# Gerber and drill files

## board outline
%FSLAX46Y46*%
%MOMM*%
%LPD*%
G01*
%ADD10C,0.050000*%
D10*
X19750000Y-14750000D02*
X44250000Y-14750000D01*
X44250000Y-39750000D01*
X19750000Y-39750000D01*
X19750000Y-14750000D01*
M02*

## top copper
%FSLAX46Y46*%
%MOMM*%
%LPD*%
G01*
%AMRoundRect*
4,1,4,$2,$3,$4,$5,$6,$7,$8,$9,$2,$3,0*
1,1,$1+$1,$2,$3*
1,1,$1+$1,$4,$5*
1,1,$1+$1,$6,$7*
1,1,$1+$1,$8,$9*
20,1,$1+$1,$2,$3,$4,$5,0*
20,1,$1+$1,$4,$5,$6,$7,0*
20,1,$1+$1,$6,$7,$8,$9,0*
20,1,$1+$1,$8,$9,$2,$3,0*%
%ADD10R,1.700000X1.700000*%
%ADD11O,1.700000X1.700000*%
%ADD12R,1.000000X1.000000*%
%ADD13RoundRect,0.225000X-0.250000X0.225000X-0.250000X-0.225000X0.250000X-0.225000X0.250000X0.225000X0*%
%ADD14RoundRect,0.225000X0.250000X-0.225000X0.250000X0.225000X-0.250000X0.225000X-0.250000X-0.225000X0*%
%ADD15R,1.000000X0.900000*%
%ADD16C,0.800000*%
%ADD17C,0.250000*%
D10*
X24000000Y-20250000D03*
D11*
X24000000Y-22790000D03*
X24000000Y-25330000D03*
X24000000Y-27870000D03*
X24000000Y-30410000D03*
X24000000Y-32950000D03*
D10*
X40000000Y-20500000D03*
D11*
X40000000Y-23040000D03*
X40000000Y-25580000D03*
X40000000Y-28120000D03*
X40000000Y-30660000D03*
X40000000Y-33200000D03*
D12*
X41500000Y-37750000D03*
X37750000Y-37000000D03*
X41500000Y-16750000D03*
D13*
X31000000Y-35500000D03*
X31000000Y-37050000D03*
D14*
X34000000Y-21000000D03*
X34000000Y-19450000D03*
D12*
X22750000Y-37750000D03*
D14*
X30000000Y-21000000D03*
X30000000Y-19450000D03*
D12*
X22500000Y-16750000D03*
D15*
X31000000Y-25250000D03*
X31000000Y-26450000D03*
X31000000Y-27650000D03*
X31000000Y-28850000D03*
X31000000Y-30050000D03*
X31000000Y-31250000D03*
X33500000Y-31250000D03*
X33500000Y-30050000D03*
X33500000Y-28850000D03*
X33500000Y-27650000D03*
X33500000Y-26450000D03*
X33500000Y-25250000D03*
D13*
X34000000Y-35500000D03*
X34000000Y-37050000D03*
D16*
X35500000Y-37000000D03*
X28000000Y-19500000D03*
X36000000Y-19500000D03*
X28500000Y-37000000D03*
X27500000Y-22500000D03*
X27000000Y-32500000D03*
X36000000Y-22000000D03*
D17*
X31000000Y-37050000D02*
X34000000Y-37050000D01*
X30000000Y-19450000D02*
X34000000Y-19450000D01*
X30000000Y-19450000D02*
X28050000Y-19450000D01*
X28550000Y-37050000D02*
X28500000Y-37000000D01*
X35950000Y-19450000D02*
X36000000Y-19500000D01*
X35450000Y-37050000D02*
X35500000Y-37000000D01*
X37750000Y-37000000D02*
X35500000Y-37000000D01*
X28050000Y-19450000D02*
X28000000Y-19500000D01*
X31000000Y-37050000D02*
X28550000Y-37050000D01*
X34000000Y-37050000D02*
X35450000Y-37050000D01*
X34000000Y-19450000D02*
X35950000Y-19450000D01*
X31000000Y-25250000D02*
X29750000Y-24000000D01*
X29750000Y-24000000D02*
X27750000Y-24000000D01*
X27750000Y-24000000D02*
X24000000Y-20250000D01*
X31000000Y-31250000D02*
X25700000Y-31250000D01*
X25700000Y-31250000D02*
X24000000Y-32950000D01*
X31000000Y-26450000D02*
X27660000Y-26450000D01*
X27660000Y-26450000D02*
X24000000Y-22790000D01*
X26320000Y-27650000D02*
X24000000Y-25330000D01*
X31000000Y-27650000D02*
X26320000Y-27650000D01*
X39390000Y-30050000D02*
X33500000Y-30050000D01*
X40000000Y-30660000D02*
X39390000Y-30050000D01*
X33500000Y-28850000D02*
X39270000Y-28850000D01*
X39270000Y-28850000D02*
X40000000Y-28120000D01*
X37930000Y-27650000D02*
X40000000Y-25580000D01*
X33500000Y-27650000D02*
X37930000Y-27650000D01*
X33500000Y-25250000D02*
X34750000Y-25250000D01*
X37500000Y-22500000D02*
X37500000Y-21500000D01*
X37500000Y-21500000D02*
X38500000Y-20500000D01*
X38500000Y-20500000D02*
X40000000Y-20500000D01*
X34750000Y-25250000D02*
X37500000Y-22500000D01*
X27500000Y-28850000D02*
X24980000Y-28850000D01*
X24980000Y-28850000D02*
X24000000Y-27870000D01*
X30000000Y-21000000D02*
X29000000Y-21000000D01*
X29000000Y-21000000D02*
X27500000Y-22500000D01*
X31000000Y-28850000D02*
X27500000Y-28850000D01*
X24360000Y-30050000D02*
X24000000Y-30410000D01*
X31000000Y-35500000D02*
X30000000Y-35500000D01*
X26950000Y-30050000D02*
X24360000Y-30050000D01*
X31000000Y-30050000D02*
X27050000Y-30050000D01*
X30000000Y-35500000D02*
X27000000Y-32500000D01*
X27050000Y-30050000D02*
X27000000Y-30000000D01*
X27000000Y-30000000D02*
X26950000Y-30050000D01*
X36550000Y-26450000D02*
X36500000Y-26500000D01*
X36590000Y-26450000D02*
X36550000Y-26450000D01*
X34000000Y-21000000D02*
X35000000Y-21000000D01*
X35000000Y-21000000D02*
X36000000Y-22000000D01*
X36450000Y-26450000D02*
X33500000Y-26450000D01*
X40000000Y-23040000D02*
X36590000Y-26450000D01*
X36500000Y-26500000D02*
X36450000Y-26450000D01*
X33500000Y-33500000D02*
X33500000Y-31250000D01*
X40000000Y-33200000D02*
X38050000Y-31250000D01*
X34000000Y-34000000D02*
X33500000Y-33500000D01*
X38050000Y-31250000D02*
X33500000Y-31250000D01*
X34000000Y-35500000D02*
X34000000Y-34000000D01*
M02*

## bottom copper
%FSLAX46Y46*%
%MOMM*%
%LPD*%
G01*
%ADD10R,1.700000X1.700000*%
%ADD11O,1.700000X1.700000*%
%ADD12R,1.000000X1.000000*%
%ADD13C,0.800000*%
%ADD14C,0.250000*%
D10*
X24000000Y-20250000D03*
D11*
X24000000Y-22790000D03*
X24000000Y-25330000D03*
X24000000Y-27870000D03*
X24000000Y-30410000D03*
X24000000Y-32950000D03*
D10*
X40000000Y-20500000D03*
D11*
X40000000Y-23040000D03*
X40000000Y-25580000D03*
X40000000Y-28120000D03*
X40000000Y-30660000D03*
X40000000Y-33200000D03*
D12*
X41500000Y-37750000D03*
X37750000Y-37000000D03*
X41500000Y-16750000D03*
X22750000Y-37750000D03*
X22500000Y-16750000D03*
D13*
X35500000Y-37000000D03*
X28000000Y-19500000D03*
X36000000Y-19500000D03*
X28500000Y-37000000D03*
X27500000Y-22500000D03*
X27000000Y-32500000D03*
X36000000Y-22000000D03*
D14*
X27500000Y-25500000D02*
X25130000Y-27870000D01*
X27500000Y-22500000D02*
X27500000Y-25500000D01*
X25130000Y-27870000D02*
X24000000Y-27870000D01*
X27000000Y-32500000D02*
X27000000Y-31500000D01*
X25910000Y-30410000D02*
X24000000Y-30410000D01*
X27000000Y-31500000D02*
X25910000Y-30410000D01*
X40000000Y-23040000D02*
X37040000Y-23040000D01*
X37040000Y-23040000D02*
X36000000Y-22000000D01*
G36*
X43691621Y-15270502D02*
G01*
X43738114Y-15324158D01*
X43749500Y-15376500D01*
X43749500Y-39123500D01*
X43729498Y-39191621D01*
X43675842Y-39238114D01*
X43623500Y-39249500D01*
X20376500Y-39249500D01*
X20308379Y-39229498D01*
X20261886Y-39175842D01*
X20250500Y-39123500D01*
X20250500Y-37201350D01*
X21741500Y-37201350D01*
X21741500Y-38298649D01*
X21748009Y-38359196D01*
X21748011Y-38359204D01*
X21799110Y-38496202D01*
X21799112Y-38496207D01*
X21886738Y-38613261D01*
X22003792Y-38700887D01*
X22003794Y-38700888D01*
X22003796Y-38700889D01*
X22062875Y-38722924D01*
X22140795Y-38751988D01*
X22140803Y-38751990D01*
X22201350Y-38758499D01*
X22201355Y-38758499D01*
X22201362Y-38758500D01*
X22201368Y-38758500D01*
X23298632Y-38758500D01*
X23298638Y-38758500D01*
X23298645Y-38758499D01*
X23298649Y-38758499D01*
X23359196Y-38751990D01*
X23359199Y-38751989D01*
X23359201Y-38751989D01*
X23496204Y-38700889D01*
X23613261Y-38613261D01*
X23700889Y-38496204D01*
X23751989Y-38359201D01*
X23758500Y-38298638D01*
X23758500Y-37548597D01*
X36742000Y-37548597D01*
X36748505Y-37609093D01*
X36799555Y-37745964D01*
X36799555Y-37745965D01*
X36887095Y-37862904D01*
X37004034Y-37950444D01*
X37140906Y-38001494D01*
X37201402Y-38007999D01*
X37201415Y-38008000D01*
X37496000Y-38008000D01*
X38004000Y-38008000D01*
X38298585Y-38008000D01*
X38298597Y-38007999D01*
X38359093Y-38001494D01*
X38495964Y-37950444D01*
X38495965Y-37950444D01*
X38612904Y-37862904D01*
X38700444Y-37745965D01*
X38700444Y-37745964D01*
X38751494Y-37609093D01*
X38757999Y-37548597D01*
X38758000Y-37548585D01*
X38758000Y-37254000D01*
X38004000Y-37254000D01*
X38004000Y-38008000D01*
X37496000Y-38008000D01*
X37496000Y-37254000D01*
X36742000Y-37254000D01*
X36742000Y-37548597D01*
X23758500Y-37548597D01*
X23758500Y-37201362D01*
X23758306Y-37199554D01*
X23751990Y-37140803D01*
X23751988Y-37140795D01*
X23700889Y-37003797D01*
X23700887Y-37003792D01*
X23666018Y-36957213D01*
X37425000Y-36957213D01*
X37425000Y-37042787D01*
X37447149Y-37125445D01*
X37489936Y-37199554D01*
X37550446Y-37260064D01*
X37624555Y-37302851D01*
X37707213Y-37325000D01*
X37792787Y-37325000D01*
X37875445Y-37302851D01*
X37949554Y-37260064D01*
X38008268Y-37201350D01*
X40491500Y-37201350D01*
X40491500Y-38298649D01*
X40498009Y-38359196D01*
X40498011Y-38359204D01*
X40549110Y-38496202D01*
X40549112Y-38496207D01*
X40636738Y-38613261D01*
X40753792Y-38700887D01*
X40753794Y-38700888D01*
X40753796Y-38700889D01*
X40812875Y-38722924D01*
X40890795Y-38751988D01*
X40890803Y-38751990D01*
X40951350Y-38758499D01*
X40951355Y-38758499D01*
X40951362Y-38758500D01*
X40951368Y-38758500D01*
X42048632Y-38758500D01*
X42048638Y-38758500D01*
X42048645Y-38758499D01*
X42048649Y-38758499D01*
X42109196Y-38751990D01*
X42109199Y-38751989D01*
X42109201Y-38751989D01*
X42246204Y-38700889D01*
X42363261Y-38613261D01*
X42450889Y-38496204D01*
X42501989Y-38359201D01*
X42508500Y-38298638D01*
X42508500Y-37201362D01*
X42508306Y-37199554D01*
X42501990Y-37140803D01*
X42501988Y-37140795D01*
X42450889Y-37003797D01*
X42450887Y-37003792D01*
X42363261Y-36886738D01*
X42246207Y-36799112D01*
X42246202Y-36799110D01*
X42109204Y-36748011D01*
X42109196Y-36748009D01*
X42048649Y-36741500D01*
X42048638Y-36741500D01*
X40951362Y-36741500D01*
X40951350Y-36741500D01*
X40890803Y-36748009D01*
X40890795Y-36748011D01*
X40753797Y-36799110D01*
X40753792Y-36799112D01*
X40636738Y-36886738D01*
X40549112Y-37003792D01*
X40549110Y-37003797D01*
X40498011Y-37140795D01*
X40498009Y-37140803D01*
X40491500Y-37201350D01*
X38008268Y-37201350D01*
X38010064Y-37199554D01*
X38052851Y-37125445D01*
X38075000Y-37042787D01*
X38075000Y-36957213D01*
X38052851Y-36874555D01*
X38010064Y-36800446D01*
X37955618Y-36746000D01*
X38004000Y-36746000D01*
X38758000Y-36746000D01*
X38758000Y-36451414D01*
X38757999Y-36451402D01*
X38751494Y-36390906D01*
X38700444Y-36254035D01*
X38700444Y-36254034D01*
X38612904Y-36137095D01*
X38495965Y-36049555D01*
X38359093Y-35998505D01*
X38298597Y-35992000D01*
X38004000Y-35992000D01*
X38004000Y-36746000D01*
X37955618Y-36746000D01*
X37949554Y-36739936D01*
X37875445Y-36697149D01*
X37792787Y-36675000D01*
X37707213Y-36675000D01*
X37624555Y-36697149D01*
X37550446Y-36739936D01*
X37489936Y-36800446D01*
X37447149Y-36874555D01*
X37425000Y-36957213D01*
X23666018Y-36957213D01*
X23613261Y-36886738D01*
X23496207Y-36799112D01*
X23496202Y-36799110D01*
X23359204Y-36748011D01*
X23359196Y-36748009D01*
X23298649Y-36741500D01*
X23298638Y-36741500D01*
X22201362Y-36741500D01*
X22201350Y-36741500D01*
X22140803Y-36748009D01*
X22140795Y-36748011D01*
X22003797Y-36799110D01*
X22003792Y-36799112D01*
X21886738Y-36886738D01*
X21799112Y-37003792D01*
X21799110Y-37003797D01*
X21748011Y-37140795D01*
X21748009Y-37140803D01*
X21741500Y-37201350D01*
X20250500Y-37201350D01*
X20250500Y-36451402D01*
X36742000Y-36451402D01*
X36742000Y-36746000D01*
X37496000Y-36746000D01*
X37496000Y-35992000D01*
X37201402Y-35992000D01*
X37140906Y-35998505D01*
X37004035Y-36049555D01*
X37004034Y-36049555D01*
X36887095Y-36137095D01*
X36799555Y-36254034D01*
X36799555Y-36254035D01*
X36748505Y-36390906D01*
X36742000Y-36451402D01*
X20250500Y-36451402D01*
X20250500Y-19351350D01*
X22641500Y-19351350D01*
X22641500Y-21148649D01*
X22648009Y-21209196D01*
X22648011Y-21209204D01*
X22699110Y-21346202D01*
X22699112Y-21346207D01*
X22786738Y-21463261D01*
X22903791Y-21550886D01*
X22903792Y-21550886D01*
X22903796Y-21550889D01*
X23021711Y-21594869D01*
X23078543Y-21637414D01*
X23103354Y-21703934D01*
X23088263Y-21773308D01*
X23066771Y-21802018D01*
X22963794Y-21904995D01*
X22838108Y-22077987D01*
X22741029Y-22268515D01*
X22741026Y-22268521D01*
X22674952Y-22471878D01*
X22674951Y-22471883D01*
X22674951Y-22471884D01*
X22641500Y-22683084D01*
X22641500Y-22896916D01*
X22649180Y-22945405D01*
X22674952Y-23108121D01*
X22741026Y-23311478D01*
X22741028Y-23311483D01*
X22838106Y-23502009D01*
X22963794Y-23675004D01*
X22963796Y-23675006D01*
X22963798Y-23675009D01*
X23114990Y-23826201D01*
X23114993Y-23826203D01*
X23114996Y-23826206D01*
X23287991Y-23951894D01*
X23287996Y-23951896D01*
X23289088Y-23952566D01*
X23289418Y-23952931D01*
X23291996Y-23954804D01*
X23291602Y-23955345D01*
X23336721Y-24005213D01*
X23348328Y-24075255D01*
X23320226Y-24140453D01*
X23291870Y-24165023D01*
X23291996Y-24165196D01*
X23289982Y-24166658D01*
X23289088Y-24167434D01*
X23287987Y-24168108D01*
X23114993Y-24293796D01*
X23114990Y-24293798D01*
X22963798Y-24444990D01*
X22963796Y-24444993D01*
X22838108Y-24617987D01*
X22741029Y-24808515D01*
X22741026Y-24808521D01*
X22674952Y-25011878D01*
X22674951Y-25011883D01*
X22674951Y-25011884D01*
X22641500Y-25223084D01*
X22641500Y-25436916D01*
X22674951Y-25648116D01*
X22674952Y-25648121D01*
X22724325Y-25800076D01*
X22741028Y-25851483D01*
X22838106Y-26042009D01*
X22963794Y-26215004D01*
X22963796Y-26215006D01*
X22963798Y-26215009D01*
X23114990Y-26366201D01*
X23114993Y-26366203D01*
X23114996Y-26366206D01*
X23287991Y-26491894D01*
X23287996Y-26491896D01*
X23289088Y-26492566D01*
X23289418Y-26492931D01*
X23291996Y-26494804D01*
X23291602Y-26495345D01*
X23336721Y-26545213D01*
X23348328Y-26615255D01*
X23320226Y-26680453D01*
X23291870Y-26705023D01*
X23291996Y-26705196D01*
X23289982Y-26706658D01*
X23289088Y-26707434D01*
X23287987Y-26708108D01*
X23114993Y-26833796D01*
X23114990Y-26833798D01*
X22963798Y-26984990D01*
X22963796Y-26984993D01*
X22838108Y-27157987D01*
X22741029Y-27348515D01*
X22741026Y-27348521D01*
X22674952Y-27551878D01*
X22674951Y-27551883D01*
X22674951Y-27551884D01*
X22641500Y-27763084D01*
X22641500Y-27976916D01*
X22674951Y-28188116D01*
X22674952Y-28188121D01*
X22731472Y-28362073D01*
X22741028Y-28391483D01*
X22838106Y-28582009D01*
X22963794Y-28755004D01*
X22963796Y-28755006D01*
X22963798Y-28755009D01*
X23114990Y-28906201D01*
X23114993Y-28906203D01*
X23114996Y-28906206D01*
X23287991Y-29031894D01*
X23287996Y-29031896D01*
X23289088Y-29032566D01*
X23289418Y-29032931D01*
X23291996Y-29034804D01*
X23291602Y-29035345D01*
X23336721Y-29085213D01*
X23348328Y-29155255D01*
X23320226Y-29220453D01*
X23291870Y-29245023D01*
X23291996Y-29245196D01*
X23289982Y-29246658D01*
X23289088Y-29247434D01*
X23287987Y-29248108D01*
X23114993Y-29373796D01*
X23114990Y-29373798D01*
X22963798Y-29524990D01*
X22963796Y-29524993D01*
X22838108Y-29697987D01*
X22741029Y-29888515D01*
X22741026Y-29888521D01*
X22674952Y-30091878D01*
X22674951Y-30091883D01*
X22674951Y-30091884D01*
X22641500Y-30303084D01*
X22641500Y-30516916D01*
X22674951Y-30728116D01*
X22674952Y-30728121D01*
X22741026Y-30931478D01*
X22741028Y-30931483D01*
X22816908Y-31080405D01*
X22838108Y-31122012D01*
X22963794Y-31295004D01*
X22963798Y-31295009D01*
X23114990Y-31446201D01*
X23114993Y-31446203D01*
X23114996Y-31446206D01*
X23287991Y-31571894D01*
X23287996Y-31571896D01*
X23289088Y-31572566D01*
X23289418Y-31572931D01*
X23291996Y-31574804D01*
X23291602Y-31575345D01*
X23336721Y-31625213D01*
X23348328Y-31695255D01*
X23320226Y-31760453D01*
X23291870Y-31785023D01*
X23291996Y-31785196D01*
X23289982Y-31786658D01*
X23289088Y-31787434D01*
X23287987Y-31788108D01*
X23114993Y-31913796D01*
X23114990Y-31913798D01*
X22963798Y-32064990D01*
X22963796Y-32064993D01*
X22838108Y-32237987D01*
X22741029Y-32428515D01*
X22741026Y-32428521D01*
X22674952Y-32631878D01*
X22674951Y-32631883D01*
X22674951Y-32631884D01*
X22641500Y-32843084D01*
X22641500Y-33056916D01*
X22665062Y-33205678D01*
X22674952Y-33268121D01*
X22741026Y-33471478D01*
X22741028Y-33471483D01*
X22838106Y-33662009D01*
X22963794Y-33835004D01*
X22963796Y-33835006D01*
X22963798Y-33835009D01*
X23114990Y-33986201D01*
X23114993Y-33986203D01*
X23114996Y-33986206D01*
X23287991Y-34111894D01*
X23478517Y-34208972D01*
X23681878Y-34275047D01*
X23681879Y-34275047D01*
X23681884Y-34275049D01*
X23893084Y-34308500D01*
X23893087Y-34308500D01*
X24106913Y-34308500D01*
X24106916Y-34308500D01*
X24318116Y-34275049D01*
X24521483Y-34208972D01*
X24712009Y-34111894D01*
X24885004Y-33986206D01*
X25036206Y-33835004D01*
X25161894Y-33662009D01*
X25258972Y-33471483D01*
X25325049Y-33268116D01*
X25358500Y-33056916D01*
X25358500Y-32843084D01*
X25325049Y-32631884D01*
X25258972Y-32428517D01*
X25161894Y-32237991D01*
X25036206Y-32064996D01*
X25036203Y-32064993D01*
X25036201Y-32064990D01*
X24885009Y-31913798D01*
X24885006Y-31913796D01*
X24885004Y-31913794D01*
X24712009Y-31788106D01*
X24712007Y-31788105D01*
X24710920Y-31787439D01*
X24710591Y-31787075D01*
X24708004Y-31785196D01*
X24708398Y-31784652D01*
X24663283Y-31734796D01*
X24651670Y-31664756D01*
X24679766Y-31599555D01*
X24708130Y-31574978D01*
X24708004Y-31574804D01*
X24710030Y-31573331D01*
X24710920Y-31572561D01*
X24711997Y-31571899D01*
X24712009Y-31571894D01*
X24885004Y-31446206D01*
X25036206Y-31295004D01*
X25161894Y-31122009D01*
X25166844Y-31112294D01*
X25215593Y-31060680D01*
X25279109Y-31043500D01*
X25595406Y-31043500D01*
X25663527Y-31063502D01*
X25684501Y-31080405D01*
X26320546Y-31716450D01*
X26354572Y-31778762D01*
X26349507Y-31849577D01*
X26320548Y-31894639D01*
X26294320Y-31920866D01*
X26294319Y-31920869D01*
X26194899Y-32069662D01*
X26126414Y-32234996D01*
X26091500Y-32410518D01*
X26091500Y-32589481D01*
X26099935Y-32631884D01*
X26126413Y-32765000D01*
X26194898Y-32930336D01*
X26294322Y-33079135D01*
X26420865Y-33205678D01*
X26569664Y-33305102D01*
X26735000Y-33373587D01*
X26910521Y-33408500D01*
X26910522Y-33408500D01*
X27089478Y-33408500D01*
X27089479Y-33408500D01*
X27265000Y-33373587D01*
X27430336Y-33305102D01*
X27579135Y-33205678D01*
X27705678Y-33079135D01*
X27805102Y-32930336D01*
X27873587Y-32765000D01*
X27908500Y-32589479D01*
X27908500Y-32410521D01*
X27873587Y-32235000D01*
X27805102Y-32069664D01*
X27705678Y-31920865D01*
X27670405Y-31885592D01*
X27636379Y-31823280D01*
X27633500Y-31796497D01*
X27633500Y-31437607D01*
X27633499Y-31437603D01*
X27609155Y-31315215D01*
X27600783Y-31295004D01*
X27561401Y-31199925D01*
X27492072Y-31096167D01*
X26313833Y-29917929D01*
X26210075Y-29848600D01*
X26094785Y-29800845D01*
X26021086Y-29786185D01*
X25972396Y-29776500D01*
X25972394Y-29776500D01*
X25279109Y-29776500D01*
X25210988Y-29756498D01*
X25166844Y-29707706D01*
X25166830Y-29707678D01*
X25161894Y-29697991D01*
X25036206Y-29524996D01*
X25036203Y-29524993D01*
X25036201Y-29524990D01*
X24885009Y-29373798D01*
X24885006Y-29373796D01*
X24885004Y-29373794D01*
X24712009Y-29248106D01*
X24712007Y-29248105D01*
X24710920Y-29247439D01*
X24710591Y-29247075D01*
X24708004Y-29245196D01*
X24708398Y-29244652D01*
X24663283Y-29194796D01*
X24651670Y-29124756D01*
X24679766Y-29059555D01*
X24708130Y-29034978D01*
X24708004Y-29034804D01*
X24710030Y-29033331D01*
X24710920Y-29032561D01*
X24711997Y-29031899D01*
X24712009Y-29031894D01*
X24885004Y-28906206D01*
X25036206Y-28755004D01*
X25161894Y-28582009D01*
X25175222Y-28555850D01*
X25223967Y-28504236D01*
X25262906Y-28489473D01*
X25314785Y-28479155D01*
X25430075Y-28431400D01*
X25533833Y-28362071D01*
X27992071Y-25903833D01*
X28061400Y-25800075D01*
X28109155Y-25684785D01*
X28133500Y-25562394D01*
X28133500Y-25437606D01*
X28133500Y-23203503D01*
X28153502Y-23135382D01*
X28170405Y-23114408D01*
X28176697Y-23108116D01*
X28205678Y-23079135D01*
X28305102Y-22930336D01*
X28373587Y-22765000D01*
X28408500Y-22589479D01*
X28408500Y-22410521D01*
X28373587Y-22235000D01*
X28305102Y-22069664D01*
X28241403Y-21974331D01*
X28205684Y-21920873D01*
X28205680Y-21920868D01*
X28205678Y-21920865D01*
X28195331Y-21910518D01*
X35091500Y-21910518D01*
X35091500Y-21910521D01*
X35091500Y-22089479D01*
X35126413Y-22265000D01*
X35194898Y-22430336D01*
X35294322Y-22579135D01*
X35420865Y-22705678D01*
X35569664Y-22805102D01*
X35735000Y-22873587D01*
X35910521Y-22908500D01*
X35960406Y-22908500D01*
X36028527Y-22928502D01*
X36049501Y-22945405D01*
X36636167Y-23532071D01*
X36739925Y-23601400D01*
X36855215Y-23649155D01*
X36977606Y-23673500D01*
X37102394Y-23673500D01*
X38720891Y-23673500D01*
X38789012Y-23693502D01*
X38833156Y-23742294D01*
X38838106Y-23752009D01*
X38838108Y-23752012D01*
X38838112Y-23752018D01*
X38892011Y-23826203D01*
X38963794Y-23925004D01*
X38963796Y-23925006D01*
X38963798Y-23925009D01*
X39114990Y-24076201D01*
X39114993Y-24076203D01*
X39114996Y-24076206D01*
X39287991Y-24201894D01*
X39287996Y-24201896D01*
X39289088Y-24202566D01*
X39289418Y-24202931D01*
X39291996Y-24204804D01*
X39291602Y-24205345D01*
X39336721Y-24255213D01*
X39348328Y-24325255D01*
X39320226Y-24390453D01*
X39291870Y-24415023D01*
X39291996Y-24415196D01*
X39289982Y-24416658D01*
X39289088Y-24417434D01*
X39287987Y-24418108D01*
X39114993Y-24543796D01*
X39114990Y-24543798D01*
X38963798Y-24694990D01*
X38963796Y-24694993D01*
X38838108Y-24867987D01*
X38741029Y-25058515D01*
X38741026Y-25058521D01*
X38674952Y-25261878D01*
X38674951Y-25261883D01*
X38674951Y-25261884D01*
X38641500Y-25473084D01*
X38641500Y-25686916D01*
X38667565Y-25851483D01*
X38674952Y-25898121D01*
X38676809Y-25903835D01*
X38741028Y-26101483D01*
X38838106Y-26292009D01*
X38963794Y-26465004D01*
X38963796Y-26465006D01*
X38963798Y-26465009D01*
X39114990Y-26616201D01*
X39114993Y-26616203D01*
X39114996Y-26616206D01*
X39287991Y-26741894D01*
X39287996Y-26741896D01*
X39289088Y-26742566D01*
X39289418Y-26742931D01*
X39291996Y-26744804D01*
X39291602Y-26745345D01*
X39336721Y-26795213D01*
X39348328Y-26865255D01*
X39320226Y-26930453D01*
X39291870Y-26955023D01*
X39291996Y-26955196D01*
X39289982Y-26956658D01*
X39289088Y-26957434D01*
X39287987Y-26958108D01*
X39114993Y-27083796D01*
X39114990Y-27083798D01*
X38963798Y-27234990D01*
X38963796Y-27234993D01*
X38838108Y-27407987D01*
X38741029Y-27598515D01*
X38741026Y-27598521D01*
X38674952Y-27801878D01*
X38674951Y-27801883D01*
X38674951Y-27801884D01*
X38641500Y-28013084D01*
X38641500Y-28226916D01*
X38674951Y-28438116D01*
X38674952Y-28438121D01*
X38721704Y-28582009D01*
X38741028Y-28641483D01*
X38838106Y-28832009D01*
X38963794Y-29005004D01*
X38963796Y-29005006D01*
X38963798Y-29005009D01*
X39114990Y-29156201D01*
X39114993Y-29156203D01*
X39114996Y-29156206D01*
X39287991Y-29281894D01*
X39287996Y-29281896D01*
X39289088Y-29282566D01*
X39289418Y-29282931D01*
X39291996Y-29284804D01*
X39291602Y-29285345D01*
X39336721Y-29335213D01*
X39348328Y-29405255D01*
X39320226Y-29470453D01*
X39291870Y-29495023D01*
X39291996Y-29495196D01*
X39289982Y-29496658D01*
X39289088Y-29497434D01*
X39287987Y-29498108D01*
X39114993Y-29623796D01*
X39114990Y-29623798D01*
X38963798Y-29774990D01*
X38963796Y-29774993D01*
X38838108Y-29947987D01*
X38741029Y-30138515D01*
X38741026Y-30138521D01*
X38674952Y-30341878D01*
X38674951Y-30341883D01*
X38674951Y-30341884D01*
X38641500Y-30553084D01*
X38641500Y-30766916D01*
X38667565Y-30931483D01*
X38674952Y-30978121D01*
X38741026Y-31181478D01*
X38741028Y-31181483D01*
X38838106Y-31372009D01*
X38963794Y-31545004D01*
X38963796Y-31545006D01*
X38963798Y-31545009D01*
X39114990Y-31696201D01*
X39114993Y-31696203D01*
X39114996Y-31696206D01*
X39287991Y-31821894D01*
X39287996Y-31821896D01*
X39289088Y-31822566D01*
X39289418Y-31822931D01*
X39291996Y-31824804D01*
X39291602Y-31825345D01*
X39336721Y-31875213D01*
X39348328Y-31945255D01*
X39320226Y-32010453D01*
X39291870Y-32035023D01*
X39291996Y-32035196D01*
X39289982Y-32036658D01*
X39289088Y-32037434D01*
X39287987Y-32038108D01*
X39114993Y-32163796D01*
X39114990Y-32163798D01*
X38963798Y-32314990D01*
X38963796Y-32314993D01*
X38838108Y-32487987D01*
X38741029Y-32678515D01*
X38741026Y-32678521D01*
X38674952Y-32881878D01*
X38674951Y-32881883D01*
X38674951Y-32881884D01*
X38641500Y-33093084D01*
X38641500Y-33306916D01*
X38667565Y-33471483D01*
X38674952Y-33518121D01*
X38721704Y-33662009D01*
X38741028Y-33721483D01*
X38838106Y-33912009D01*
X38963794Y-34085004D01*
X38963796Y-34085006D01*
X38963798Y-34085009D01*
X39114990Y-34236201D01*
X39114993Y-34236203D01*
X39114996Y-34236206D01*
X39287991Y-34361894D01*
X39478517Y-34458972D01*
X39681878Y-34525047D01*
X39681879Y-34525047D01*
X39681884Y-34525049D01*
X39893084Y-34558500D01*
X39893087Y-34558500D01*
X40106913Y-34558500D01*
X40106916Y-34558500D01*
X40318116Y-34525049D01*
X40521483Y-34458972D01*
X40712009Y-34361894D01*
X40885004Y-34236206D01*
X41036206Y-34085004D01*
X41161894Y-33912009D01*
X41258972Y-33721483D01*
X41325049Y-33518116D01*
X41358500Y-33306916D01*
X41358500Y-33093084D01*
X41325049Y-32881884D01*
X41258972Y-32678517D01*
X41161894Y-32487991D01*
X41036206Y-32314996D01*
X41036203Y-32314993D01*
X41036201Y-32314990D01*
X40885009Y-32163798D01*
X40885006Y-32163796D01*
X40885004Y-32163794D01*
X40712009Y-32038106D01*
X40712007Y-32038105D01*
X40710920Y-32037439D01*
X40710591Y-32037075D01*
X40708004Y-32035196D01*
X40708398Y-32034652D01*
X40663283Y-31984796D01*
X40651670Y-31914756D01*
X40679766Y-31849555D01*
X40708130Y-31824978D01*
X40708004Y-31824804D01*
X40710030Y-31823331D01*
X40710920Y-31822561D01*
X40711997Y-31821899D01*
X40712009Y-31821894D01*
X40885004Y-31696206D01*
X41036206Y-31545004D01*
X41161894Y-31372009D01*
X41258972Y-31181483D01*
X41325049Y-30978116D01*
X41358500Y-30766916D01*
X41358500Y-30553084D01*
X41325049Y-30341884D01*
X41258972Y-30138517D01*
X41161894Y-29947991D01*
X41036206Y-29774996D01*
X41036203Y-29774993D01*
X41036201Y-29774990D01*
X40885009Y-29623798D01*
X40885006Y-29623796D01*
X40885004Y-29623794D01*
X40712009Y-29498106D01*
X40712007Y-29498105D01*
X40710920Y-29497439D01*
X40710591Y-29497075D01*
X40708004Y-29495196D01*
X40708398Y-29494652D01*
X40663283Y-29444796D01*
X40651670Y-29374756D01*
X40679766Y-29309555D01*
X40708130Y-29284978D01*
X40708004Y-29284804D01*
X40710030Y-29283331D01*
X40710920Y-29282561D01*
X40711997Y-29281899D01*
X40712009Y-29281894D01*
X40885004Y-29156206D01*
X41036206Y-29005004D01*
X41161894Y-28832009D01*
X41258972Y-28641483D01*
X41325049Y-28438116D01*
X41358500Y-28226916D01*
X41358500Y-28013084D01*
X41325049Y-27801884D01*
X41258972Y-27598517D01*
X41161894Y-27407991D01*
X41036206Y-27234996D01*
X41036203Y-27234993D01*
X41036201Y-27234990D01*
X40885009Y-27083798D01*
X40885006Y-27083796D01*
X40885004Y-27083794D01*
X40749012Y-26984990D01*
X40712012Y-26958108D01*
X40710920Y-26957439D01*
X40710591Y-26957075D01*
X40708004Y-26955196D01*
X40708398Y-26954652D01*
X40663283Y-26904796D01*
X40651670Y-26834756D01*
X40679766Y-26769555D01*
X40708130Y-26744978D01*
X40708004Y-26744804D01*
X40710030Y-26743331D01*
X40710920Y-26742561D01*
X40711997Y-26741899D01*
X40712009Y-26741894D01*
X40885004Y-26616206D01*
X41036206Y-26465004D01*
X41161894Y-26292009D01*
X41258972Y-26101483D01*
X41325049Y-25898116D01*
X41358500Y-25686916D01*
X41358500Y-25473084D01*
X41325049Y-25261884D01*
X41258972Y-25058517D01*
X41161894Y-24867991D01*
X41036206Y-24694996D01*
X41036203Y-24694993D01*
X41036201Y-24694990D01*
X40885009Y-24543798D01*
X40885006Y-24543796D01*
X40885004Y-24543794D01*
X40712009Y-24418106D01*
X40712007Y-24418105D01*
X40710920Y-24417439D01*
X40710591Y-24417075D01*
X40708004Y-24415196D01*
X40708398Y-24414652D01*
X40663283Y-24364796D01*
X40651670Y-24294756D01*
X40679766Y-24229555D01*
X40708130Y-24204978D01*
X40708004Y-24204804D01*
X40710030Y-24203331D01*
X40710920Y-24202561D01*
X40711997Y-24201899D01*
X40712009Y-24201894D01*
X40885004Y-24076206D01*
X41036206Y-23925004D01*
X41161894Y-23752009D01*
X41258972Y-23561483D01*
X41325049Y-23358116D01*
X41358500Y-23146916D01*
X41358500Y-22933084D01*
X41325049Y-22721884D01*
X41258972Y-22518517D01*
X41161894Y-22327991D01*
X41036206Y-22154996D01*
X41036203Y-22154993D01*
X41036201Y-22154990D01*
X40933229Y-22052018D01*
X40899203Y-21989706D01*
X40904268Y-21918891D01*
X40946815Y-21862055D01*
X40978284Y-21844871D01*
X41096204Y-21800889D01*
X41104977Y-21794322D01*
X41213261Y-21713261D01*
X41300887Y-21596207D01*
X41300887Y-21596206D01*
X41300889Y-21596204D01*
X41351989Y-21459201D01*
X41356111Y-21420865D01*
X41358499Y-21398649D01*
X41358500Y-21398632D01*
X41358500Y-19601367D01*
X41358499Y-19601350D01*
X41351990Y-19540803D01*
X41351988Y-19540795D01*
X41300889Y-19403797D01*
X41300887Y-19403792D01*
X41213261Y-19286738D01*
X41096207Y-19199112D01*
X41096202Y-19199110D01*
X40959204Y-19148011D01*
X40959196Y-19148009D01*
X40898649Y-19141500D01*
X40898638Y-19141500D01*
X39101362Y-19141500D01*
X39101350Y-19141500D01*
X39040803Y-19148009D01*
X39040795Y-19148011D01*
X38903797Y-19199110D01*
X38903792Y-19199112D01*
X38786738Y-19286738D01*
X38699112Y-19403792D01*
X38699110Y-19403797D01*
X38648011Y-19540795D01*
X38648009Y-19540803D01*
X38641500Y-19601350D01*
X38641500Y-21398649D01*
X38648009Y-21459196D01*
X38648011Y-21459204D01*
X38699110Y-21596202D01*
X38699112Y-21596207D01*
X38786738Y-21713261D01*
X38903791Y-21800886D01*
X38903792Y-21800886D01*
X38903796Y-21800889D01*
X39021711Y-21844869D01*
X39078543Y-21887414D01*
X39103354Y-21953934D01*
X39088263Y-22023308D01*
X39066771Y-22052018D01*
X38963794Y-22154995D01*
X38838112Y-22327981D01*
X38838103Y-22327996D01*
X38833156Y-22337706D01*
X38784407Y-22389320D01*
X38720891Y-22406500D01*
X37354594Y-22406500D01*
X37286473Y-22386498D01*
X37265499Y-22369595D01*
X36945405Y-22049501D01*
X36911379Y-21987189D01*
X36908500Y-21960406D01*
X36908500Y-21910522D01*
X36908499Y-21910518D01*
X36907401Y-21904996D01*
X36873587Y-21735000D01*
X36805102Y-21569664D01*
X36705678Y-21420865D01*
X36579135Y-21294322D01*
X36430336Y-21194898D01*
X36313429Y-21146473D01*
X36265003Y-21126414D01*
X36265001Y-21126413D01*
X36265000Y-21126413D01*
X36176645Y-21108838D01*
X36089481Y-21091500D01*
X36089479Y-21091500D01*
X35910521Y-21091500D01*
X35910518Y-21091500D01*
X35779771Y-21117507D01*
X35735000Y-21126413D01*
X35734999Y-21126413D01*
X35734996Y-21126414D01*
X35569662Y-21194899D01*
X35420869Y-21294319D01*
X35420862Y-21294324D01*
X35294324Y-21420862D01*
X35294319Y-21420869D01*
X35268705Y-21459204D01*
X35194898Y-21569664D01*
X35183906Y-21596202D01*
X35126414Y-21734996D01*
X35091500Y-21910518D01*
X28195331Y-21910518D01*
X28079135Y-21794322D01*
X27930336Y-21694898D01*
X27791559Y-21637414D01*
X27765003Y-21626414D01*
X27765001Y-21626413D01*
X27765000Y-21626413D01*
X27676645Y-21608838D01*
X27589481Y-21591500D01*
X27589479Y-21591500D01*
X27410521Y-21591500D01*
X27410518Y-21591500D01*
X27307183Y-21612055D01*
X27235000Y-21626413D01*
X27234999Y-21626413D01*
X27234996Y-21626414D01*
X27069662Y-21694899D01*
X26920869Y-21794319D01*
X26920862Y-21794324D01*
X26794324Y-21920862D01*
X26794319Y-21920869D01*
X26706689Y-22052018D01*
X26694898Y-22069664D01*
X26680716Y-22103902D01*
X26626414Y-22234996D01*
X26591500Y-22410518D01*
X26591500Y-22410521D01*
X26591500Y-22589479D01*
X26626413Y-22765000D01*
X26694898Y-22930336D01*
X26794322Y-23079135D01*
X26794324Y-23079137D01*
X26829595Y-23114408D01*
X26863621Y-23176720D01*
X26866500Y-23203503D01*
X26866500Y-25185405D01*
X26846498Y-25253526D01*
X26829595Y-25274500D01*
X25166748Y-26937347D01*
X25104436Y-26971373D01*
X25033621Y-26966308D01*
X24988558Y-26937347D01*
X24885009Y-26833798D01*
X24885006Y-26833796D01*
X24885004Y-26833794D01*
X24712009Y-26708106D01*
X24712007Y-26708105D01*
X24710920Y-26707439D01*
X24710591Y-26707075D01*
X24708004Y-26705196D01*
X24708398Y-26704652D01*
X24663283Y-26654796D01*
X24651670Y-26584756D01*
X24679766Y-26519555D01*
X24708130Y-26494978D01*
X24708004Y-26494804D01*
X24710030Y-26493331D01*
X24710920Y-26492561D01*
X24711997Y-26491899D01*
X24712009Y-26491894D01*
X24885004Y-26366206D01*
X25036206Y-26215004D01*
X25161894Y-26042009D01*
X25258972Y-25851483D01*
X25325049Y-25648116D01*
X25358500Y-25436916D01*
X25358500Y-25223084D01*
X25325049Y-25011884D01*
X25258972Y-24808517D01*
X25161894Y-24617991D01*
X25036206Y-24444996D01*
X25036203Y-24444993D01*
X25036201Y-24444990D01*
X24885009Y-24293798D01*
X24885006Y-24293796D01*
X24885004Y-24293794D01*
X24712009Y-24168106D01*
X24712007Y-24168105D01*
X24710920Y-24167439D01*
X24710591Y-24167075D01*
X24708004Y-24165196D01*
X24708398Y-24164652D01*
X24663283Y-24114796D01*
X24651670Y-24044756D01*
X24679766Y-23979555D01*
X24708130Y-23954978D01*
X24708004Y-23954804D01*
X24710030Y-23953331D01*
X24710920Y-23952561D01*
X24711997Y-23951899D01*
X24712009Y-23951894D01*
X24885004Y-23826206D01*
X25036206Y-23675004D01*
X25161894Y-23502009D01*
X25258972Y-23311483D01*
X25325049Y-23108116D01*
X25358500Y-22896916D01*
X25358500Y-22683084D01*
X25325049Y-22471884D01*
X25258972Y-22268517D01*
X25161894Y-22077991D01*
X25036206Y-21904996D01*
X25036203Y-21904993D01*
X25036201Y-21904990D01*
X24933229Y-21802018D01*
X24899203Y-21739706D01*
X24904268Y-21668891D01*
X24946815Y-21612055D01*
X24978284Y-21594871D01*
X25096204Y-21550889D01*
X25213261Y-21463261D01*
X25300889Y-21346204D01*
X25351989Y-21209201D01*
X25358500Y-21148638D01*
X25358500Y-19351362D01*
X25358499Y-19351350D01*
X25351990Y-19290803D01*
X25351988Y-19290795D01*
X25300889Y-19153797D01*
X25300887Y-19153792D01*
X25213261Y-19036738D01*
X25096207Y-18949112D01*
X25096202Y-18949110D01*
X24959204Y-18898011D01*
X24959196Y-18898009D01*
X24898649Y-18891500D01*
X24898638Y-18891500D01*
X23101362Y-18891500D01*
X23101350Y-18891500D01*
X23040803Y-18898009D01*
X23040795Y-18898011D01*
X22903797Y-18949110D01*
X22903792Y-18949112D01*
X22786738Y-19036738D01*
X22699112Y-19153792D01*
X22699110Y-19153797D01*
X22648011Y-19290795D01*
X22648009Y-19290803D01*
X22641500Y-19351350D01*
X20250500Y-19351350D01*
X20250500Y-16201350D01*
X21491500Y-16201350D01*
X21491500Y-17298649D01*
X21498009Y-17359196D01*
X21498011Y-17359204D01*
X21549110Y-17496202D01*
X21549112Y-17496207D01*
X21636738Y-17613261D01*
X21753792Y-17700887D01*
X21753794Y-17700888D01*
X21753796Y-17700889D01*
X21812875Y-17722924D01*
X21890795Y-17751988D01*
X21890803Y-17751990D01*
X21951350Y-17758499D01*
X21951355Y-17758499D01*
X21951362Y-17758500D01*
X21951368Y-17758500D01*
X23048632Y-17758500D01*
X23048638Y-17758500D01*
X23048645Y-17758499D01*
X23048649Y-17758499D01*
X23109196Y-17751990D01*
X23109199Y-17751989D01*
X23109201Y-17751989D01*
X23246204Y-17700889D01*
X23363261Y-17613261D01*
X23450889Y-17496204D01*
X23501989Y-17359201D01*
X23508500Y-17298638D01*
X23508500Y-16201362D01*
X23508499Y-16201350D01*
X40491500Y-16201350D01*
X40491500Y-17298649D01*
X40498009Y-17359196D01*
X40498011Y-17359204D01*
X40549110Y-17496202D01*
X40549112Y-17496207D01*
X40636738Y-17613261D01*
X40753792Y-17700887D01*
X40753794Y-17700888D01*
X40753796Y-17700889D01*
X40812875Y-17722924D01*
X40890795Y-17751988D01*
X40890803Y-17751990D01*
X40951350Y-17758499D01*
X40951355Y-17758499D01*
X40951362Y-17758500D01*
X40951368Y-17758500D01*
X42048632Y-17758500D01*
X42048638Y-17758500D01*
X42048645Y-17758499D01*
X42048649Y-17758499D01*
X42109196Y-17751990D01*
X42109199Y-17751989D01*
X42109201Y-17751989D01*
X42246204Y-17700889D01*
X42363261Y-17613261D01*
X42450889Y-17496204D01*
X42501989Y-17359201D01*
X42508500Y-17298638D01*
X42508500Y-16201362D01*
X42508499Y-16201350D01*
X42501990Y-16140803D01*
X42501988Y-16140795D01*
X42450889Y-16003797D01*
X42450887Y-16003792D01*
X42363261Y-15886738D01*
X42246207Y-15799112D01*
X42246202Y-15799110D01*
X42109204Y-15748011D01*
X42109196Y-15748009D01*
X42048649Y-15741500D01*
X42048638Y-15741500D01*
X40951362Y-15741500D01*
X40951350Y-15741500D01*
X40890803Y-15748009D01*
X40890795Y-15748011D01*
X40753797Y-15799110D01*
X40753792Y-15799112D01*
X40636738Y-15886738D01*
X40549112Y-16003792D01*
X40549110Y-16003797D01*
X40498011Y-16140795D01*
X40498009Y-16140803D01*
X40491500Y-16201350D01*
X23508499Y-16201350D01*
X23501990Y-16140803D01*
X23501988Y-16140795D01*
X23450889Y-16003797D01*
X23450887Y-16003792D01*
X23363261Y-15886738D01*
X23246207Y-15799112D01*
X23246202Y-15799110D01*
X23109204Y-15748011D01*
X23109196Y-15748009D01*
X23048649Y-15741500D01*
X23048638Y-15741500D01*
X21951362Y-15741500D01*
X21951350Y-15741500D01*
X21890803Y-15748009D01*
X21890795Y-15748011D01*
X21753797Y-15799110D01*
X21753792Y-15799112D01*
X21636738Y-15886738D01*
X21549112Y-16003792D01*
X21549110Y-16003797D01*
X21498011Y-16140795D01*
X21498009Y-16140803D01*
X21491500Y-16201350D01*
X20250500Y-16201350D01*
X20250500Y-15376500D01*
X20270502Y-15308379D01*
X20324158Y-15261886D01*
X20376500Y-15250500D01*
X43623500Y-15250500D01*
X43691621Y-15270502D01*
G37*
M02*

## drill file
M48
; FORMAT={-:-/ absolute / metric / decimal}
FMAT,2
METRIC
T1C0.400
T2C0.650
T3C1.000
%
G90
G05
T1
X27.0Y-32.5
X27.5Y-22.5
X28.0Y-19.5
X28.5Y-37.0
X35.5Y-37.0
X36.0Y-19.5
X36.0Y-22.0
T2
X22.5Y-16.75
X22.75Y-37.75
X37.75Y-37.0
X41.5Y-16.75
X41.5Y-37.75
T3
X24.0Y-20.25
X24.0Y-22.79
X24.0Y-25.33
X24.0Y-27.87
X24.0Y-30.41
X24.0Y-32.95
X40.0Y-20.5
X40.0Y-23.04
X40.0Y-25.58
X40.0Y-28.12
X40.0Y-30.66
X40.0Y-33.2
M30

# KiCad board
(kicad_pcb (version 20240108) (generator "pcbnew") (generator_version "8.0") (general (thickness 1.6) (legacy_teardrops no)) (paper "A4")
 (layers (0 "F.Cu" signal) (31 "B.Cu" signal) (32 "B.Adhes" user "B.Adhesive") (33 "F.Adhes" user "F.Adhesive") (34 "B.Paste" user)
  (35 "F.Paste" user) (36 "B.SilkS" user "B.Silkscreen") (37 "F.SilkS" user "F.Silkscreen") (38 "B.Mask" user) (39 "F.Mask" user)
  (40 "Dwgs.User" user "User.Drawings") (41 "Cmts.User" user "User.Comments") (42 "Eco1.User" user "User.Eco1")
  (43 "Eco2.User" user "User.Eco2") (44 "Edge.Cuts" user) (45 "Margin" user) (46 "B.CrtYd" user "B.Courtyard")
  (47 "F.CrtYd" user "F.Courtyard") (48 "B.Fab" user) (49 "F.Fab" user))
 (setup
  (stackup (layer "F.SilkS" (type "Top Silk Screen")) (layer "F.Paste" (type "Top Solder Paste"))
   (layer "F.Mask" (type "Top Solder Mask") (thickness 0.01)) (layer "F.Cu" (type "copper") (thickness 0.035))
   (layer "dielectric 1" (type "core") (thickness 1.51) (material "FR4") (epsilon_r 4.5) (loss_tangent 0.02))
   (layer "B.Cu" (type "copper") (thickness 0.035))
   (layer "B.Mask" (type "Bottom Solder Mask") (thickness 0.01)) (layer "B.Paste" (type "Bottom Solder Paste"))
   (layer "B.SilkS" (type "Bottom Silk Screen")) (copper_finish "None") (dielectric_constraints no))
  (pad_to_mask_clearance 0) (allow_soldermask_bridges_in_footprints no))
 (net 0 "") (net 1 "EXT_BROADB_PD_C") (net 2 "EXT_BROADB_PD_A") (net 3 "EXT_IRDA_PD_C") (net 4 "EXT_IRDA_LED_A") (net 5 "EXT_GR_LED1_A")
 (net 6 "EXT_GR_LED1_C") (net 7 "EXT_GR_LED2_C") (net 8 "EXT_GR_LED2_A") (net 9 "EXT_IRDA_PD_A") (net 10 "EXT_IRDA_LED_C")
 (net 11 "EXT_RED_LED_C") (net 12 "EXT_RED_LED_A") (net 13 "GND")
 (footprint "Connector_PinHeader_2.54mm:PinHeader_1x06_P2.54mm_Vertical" (layer "F.Cu") (at 24 20.25)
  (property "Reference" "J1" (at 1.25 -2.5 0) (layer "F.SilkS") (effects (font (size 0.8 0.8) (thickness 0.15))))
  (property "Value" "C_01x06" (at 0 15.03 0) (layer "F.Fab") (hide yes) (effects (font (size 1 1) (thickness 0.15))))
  (pad "1" thru_hole rect (at 0 0) (size 1.7 1.7) (drill 1) (layers "*.Cu" "*.Mask") (remove_unused_layers no) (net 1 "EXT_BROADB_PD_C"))
  (pad "2" thru_hole oval (at 0 2.54) (size 1.7 1.7) (drill 1) (layers "*.Cu" "*.Mask") (remove_unused_layers no) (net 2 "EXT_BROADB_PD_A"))
  (pad "3" thru_hole oval (at 0 5.08) (size 1.7 1.7) (drill 1) (layers "*.Cu" "*.Mask") (remove_unused_layers no) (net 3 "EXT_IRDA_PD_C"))
  (pad "4" thru_hole oval (at 0 7.62) (size 1.7 1.7) (drill 1) (layers "*.Cu" "*.Mask") (remove_unused_layers no) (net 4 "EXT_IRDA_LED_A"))
  (pad "5" thru_hole oval (at 0 10.16) (size 1.7 1.7) (drill 1) (layers "*.Cu" "*.Mask") (remove_unused_layers no) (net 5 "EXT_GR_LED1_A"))
  (pad "6" thru_hole oval (at 0 12.7) (size 1.7 1.7) (drill 1) (layers "*.Cu" "*.Mask") (remove_unused_layers no) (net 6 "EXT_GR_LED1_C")))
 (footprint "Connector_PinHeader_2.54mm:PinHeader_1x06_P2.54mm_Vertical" (layer "F.Cu") (at 40 20.5)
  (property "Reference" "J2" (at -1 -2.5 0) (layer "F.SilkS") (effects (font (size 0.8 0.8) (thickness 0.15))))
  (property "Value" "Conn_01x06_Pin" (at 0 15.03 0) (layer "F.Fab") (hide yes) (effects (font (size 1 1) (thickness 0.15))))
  (pad "1" thru_hole rect (at 0 0) (size 1.7 1.7) (drill 1) (layers "*.Cu" "*.Mask") (remove_unused_layers no) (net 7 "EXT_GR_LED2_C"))
  (pad "2" thru_hole oval (at 0 2.54) (size 1.7 1.7) (drill 1) (layers "*.Cu" "*.Mask") (remove_unused_layers no) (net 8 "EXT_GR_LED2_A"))
  (pad "3" thru_hole oval (at 0 5.08) (size 1.7 1.7) (drill 1) (layers "*.Cu" "*.Mask") (remove_unused_layers no) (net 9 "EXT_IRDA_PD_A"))
  (pad "4" thru_hole oval (at 0 7.62) (size 1.7 1.7) (drill 1) (layers "*.Cu" "*.Mask") (remove_unused_layers no) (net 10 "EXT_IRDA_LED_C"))
  (pad "5" thru_hole oval (at 0 10.16) (size 1.7 1.7) (drill 1) (layers "*.Cu" "*.Mask") (remove_unused_layers no) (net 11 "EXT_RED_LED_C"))
  (pad "6" thru_hole oval (at 0 12.7) (size 1.7 1.7) (drill 1) (layers "*.Cu" "*.Mask") (remove_unused_layers no) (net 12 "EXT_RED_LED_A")))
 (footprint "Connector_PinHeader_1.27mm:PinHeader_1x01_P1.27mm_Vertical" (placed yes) (layer "F.Cu") (at 41.5 37.75 180)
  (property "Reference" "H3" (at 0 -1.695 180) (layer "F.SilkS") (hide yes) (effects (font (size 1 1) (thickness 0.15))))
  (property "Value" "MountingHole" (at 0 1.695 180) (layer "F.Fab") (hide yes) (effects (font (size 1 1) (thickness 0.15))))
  (pad "1" thru_hole rect (at 0 0 180) (size 1 1) (drill 0.65) (layers "*.Cu" "*.Mask") (remove_unused_layers no)))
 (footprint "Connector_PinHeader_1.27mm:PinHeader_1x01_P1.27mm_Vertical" (layer "F.Cu") (at 37.75 37)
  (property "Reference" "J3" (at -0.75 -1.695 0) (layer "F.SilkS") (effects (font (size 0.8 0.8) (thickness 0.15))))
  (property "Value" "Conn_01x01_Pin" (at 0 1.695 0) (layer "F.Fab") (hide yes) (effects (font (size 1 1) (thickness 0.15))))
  (pad "1" thru_hole rect (at 0 0) (size 1 1) (drill 0.65) (layers "*.Cu" "*.Mask") (remove_unused_layers no) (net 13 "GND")))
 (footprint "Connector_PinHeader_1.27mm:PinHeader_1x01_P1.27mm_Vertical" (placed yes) (layer "F.Cu") (at 41.5 16.75)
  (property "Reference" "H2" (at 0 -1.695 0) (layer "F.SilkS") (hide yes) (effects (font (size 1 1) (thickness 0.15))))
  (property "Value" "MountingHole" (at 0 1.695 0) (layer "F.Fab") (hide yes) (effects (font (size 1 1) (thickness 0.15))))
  (pad "1" thru_hole rect (at 0 0) (size 1 1) (drill 0.65) (layers "*.Cu" "*.Mask") (remove_unused_layers no)))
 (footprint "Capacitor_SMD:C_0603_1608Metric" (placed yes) (layer "F.Cu") (at 31 36.275 -90)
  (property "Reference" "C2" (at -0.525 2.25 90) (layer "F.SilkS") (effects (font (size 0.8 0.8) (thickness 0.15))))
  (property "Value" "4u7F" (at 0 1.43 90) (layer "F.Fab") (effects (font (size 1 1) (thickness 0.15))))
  (pad "1" smd roundrect (at -0.775 0 270) (size 0.9 0.95) (layers "F.Cu" "F.Paste" "F.Mask") (roundrect_rratio 0.25)
   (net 5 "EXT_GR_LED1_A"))
  (pad "2" smd roundrect (at 0.775 0 270) (size 0.9 0.95) (layers "F.Cu" "F.Paste" "F.Mask") (roundrect_rratio 0.25) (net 13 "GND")))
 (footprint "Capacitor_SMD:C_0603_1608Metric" (layer "F.Cu") (at 34 20.225 90)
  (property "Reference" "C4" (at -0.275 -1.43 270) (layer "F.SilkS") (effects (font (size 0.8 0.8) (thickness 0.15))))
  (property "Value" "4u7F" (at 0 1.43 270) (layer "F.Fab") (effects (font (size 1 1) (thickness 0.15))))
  (pad "1" smd roundrect (at -0.775 0 90) (size 0.9 0.95) (layers "F.Cu" "F.Paste" "F.Mask") (roundrect_rratio 0.25) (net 8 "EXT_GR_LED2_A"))
  (pad "2" smd roundrect (at 0.775 0 90) (size 0.9 0.95) (layers "F.Cu" "F.Paste" "F.Mask") (roundrect_rratio 0.25) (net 13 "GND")))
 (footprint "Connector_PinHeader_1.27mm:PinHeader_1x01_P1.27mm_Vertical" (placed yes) (layer "F.Cu") (at 22.75 37.75 180)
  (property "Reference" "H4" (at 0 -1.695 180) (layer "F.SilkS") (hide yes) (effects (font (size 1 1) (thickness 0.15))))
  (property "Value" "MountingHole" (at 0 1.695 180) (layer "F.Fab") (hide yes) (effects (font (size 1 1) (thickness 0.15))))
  (pad "1" thru_hole rect (at 0 0 180) (size 1 1) (drill 0.65) (layers "*.Cu" "*.Mask") (remove_unused_layers no)))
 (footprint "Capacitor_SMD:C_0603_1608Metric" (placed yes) (layer "F.Cu") (at 30 20.225 90)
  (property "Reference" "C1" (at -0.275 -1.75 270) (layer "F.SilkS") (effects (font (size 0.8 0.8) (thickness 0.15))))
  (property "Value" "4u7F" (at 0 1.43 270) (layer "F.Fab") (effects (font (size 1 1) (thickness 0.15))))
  (pad "1" smd roundrect (at -0.775 0 90) (size 0.9 0.95) (layers "F.Cu" "F.Paste" "F.Mask") (roundrect_rratio 0.25)
   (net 4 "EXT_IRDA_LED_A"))
  (pad "2" smd roundrect (at 0.775 0 90) (size 0.9 0.95) (layers "F.Cu" "F.Paste" "F.Mask") (roundrect_rratio 0.25) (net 13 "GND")))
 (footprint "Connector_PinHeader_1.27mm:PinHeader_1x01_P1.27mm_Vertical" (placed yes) (layer "F.Cu") (at 22.5 16.75)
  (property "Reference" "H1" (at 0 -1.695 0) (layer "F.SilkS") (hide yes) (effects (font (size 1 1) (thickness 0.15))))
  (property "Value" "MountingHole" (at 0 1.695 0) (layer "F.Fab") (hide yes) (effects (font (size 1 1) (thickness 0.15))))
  (pad "1" thru_hole rect (at 0 0) (size 1 1) (drill 0.65) (layers "*.Cu" "*.Mask") (remove_unused_layers no)))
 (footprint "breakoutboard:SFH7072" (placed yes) (layer "F.Cu") (at 31.875 28.25 -90)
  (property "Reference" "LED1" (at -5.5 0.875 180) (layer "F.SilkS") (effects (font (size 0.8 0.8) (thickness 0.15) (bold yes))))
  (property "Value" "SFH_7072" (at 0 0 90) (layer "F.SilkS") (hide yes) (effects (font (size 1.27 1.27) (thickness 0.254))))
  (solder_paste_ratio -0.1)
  (pad "1" smd rect (at -3 0.875 270) (size 0.9 1) (layers "F.Cu" "F.Paste" "F.Mask") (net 1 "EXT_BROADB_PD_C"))
  (pad "2" smd rect (at -1.8 0.875 270) (size 0.9 1) (layers "F.Cu" "F.Paste" "F.Mask") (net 2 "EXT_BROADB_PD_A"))
  (pad "3" smd rect (at -0.6 0.875 270) (size 0.9 1) (layers "F.Cu" "F.Paste" "F.Mask") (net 3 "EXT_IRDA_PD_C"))
  (pad "4" smd rect (at 0.6 0.875 270) (size 0.9 1) (layers "F.Cu" "F.Paste" "F.Mask") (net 4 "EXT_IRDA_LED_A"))
  (pad "5" smd rect (at 1.8 0.875 270) (size 0.9 1) (layers "F.Cu" "F.Paste" "F.Mask") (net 5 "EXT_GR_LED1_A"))
  (pad "6" smd rect (at 3 0.875 270) (size 0.9 1) (layers "F.Cu" "F.Paste" "F.Mask") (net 6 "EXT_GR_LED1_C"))
  (pad "7" smd rect (at 3 -1.625 270) (size 0.9 1) (layers "F.Cu" "F.Paste" "F.Mask") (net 12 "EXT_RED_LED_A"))
  (pad "8" smd rect (at 1.8 -1.625 270) (size 0.9 1) (layers "F.Cu" "F.Paste" "F.Mask") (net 11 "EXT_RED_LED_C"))
  (pad "9" smd rect (at 0.6 -1.625 270) (size 0.9 1) (layers "F.Cu" "F.Paste" "F.Mask") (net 10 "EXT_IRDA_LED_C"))
  (pad "10" smd rect (at -0.6 -1.625 270) (size 0.9 1) (layers "F.Cu" "F.Paste" "F.Mask") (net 9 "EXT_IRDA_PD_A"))
  (pad "11" smd rect (at -1.8 -1.625 270) (size 0.9 1) (layers "F.Cu" "F.Paste" "F.Mask") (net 8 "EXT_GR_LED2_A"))
  (pad "12" smd rect (at -3 -1.625 270) (size 0.9 1) (layers "F.Cu" "F.Paste" "F.Mask") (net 7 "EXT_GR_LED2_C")))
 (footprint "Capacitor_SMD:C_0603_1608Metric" (layer "F.Cu") (at 34 36.275 -90)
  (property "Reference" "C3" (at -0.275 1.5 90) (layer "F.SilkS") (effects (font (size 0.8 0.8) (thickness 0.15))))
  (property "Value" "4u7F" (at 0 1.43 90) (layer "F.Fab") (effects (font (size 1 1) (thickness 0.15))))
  (pad "1" smd roundrect (at -0.775 0 270) (size 0.9 0.95) (layers "F.Cu" "F.Paste" "F.Mask") (roundrect_rratio 0.25)
   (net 12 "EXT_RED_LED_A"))
  (pad "2" smd roundrect (at 0.775 0 270) (size 0.9 0.95) (layers "F.Cu" "F.Paste" "F.Mask") (roundrect_rratio 0.25) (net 13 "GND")))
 (gr_rect (start 19.75 14.75) (end 44.25 39.75) (stroke (width 0.05) (type solid)) (fill none) (layer "Edge.Cuts"))
 (segment (start 31 37.05) (end 34 37.05) (width 0.25) (layer "F.Cu") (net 13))
 (segment (start 30 19.45) (end 34 19.45) (width 0.25) (layer "F.Cu") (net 13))
 (segment (start 30 19.45) (end 28.05 19.45) (width 0.25) (layer "F.Cu") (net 13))
 (segment (start 28.55 37.05) (end 28.5 37) (width 0.25) (layer "F.Cu") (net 13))
 (segment (start 35.95 19.45) (end 36 19.5) (width 0.25) (layer "F.Cu") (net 13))
 (segment (start 35.45 37.05) (end 35.5 37) (width 0.25) (layer "F.Cu") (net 13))
 (segment (start 37.75 37) (end 35.5 37) (width 0.25) (layer "F.Cu") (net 13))
 (segment (start 28.05 19.45) (end 28 19.5) (width 0.25) (layer "F.Cu") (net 13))
 (segment (start 31 37.05) (end 28.55 37.05) (width 0.25) (layer "F.Cu") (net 13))
 (segment (start 34 37.05) (end 35.45 37.05) (width 0.25) (layer "F.Cu") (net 13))
 (segment (start 34 19.45) (end 35.95 19.45) (width 0.25) (layer "F.Cu") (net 13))
 (via (at 35.5 37) (size 0.8) (drill 0.4) (layers "F.Cu" "B.Cu") (free yes) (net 13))
 (via (at 28 19.5) (size 0.8) (drill 0.4) (layers "F.Cu" "B.Cu") (free yes) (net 13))
 (via (at 36 19.5) (size 0.8) (drill 0.4) (layers "F.Cu" "B.Cu") (free yes) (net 13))
 (via (at 28.5 37) (size 0.8) (drill 0.4) (layers "F.Cu" "B.Cu") (free yes) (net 13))
 (segment (start 31 25.25) (end 29.75 24) (width 0.25) (layer "F.Cu") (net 1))
 (segment (start 29.75 24) (end 27.75 24) (width 0.25) (layer "F.Cu") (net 1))
 (segment (start 27.75 24) (end 24 20.25) (width 0.25) (layer "F.Cu") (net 1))
 (segment (start 31 31.25) (end 25.7 31.25) (width 0.25) (layer "F.Cu") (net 6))
 (segment (start 25.7 31.25) (end 24 32.95) (width 0.25) (layer "F.Cu") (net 6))
 (segment (start 31 26.45) (end 27.66 26.45) (width 0.25) (layer "F.Cu") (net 2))
 (segment (start 27.66 26.45) (end 24 22.79) (width 0.25) (layer "F.Cu") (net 2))
 (segment (start 26.32 27.65) (end 24 25.33) (width 0.25) (layer "F.Cu") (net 3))
 (segment (start 31 27.65) (end 26.32 27.65) (width 0.25) (layer "F.Cu") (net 3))
 (segment (start 39.39 30.05) (end 33.5 30.05) (width 0.25) (layer "F.Cu") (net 11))
 (segment (start 40 30.66) (end 39.39 30.05) (width 0.25) (layer "F.Cu") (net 11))
 (segment (start 33.5 28.85) (end 39.27 28.85) (width 0.25) (layer "F.Cu") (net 10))
 (segment (start 39.27 28.85) (end 40 28.12) (width 0.25) (layer "F.Cu") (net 10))
 (segment (start 37.93 27.65) (end 40 25.58) (width 0.25) (layer "F.Cu") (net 9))
 (segment (start 33.5 27.65) (end 37.93 27.65) (width 0.25) (layer "F.Cu") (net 9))
 (segment (start 33.5 25.25) (end 34.75 25.25) (width 0.25) (layer "F.Cu") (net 7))
 (segment (start 37.5 22.5) (end 37.5 21.5) (width 0.25) (layer "F.Cu") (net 7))
 (segment (start 37.5 21.5) (end 38.5 20.5) (width 0.25) (layer "F.Cu") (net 7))
 (segment (start 38.5 20.5) (end 40 20.5) (width 0.25) (layer "F.Cu") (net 7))
 (segment (start 34.75 25.25) (end 37.5 22.5) (width 0.25) (layer "F.Cu") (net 7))
 (segment (start 27.5 28.85) (end 24.98 28.85) (width 0.25) (layer "F.Cu") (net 4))
 (segment (start 24.98 28.85) (end 24 27.87) (width 0.25) (layer "F.Cu") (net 4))
 (segment (start 30 21) (end 29 21) (width 0.25) (layer "F.Cu") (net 4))
 (segment (start 29 21) (end 27.5 22.5) (width 0.25) (layer "F.Cu") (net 4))
 (segment (start 31 28.85) (end 27.5 28.85) (width 0.25) (layer "F.Cu") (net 4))
 (via (at 27.5 22.5) (size 0.8) (drill 0.4) (layers "F.Cu" "B.Cu") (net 4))
 (segment (start 27.5 25.5) (end 25.13 27.87) (width 0.25) (layer "B.Cu") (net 4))
 (segment (start 27.5 22.5) (end 27.5 25.5) (width 0.25) (layer "B.Cu") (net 4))
 (segment (start 25.13 27.87) (end 24 27.87) (width 0.25) (layer "B.Cu") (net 4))
 (segment (start 24.36 30.05) (end 24 30.41) (width 0.25) (layer "F.Cu") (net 5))
 (segment (start 31 35.5) (end 30 35.5) (width 0.25) (layer "F.Cu") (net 5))
 (segment (start 26.95 30.05) (end 24.36 30.05) (width 0.25) (layer "F.Cu") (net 5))
 (segment (start 31 30.05) (end 27.05 30.05) (width 0.25) (layer "F.Cu") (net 5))
 (segment (start 30 35.5) (end 27 32.5) (width 0.25) (layer "F.Cu") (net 5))
 (segment (start 27.05 30.05) (end 27 30) (width 0.25) (layer "F.Cu") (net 5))
 (segment (start 27 30) (end 26.95 30.05) (width 0.25) (layer "F.Cu") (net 5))
 (via (at 27 32.5) (size 0.8) (drill 0.4) (layers "F.Cu" "B.Cu") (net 5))
 (segment (start 27 32.5) (end 27 31.5) (width 0.25) (layer "B.Cu") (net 5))
 (segment (start 25.91 30.41) (end 24 30.41) (width 0.25) (layer "B.Cu") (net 5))
 (segment (start 27 31.5) (end 25.91 30.41) (width 0.25) (layer "B.Cu") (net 5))
 (segment (start 36.55 26.45) (end 36.5 26.5) (width 0.25) (layer "F.Cu") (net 8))
 (segment (start 36.59 26.45) (end 36.55 26.45) (width 0.25) (layer "F.Cu") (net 8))
 (segment (start 34 21) (end 35 21) (width 0.25) (layer "F.Cu") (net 8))
 (segment (start 35 21) (end 36 22) (width 0.25) (layer "F.Cu") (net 8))
 (segment (start 36.45 26.45) (end 33.5 26.45) (width 0.25) (layer "F.Cu") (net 8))
 (segment (start 40 23.04) (end 36.59 26.45) (width 0.25) (layer "F.Cu") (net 8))
 (segment (start 36.5 26.5) (end 36.45 26.45) (width 0.25) (layer "F.Cu") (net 8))
 (via (at 36 22) (size 0.8) (drill 0.4) (layers "F.Cu" "B.Cu") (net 8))
 (segment (start 40 23.04) (end 37.04 23.04) (width 0.25) (layer "B.Cu") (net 8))
 (segment (start 37.04 23.04) (end 36 22) (width 0.25) (layer "B.Cu") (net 8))
 (segment (start 33.5 33.5) (end 33.5 31.25) (width 0.25) (layer "F.Cu") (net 12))
 (segment (start 40 33.2) (end 38.05 31.25) (width 0.25) (layer "F.Cu") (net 12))
 (segment (start 34 34) (end 33.5 33.5) (width 0.25) (layer "F.Cu") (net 12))
 (segment (start 38.05 31.25) (end 33.5 31.25) (width 0.25) (layer "F.Cu") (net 12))
 (segment (start 34 35.5) (end 34 34) (width 0.25) (layer "F.Cu") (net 12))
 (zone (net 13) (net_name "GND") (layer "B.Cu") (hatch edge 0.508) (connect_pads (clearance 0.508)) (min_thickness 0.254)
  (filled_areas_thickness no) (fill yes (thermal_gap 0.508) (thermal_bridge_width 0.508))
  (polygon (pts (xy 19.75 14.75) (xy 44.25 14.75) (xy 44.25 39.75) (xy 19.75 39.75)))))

